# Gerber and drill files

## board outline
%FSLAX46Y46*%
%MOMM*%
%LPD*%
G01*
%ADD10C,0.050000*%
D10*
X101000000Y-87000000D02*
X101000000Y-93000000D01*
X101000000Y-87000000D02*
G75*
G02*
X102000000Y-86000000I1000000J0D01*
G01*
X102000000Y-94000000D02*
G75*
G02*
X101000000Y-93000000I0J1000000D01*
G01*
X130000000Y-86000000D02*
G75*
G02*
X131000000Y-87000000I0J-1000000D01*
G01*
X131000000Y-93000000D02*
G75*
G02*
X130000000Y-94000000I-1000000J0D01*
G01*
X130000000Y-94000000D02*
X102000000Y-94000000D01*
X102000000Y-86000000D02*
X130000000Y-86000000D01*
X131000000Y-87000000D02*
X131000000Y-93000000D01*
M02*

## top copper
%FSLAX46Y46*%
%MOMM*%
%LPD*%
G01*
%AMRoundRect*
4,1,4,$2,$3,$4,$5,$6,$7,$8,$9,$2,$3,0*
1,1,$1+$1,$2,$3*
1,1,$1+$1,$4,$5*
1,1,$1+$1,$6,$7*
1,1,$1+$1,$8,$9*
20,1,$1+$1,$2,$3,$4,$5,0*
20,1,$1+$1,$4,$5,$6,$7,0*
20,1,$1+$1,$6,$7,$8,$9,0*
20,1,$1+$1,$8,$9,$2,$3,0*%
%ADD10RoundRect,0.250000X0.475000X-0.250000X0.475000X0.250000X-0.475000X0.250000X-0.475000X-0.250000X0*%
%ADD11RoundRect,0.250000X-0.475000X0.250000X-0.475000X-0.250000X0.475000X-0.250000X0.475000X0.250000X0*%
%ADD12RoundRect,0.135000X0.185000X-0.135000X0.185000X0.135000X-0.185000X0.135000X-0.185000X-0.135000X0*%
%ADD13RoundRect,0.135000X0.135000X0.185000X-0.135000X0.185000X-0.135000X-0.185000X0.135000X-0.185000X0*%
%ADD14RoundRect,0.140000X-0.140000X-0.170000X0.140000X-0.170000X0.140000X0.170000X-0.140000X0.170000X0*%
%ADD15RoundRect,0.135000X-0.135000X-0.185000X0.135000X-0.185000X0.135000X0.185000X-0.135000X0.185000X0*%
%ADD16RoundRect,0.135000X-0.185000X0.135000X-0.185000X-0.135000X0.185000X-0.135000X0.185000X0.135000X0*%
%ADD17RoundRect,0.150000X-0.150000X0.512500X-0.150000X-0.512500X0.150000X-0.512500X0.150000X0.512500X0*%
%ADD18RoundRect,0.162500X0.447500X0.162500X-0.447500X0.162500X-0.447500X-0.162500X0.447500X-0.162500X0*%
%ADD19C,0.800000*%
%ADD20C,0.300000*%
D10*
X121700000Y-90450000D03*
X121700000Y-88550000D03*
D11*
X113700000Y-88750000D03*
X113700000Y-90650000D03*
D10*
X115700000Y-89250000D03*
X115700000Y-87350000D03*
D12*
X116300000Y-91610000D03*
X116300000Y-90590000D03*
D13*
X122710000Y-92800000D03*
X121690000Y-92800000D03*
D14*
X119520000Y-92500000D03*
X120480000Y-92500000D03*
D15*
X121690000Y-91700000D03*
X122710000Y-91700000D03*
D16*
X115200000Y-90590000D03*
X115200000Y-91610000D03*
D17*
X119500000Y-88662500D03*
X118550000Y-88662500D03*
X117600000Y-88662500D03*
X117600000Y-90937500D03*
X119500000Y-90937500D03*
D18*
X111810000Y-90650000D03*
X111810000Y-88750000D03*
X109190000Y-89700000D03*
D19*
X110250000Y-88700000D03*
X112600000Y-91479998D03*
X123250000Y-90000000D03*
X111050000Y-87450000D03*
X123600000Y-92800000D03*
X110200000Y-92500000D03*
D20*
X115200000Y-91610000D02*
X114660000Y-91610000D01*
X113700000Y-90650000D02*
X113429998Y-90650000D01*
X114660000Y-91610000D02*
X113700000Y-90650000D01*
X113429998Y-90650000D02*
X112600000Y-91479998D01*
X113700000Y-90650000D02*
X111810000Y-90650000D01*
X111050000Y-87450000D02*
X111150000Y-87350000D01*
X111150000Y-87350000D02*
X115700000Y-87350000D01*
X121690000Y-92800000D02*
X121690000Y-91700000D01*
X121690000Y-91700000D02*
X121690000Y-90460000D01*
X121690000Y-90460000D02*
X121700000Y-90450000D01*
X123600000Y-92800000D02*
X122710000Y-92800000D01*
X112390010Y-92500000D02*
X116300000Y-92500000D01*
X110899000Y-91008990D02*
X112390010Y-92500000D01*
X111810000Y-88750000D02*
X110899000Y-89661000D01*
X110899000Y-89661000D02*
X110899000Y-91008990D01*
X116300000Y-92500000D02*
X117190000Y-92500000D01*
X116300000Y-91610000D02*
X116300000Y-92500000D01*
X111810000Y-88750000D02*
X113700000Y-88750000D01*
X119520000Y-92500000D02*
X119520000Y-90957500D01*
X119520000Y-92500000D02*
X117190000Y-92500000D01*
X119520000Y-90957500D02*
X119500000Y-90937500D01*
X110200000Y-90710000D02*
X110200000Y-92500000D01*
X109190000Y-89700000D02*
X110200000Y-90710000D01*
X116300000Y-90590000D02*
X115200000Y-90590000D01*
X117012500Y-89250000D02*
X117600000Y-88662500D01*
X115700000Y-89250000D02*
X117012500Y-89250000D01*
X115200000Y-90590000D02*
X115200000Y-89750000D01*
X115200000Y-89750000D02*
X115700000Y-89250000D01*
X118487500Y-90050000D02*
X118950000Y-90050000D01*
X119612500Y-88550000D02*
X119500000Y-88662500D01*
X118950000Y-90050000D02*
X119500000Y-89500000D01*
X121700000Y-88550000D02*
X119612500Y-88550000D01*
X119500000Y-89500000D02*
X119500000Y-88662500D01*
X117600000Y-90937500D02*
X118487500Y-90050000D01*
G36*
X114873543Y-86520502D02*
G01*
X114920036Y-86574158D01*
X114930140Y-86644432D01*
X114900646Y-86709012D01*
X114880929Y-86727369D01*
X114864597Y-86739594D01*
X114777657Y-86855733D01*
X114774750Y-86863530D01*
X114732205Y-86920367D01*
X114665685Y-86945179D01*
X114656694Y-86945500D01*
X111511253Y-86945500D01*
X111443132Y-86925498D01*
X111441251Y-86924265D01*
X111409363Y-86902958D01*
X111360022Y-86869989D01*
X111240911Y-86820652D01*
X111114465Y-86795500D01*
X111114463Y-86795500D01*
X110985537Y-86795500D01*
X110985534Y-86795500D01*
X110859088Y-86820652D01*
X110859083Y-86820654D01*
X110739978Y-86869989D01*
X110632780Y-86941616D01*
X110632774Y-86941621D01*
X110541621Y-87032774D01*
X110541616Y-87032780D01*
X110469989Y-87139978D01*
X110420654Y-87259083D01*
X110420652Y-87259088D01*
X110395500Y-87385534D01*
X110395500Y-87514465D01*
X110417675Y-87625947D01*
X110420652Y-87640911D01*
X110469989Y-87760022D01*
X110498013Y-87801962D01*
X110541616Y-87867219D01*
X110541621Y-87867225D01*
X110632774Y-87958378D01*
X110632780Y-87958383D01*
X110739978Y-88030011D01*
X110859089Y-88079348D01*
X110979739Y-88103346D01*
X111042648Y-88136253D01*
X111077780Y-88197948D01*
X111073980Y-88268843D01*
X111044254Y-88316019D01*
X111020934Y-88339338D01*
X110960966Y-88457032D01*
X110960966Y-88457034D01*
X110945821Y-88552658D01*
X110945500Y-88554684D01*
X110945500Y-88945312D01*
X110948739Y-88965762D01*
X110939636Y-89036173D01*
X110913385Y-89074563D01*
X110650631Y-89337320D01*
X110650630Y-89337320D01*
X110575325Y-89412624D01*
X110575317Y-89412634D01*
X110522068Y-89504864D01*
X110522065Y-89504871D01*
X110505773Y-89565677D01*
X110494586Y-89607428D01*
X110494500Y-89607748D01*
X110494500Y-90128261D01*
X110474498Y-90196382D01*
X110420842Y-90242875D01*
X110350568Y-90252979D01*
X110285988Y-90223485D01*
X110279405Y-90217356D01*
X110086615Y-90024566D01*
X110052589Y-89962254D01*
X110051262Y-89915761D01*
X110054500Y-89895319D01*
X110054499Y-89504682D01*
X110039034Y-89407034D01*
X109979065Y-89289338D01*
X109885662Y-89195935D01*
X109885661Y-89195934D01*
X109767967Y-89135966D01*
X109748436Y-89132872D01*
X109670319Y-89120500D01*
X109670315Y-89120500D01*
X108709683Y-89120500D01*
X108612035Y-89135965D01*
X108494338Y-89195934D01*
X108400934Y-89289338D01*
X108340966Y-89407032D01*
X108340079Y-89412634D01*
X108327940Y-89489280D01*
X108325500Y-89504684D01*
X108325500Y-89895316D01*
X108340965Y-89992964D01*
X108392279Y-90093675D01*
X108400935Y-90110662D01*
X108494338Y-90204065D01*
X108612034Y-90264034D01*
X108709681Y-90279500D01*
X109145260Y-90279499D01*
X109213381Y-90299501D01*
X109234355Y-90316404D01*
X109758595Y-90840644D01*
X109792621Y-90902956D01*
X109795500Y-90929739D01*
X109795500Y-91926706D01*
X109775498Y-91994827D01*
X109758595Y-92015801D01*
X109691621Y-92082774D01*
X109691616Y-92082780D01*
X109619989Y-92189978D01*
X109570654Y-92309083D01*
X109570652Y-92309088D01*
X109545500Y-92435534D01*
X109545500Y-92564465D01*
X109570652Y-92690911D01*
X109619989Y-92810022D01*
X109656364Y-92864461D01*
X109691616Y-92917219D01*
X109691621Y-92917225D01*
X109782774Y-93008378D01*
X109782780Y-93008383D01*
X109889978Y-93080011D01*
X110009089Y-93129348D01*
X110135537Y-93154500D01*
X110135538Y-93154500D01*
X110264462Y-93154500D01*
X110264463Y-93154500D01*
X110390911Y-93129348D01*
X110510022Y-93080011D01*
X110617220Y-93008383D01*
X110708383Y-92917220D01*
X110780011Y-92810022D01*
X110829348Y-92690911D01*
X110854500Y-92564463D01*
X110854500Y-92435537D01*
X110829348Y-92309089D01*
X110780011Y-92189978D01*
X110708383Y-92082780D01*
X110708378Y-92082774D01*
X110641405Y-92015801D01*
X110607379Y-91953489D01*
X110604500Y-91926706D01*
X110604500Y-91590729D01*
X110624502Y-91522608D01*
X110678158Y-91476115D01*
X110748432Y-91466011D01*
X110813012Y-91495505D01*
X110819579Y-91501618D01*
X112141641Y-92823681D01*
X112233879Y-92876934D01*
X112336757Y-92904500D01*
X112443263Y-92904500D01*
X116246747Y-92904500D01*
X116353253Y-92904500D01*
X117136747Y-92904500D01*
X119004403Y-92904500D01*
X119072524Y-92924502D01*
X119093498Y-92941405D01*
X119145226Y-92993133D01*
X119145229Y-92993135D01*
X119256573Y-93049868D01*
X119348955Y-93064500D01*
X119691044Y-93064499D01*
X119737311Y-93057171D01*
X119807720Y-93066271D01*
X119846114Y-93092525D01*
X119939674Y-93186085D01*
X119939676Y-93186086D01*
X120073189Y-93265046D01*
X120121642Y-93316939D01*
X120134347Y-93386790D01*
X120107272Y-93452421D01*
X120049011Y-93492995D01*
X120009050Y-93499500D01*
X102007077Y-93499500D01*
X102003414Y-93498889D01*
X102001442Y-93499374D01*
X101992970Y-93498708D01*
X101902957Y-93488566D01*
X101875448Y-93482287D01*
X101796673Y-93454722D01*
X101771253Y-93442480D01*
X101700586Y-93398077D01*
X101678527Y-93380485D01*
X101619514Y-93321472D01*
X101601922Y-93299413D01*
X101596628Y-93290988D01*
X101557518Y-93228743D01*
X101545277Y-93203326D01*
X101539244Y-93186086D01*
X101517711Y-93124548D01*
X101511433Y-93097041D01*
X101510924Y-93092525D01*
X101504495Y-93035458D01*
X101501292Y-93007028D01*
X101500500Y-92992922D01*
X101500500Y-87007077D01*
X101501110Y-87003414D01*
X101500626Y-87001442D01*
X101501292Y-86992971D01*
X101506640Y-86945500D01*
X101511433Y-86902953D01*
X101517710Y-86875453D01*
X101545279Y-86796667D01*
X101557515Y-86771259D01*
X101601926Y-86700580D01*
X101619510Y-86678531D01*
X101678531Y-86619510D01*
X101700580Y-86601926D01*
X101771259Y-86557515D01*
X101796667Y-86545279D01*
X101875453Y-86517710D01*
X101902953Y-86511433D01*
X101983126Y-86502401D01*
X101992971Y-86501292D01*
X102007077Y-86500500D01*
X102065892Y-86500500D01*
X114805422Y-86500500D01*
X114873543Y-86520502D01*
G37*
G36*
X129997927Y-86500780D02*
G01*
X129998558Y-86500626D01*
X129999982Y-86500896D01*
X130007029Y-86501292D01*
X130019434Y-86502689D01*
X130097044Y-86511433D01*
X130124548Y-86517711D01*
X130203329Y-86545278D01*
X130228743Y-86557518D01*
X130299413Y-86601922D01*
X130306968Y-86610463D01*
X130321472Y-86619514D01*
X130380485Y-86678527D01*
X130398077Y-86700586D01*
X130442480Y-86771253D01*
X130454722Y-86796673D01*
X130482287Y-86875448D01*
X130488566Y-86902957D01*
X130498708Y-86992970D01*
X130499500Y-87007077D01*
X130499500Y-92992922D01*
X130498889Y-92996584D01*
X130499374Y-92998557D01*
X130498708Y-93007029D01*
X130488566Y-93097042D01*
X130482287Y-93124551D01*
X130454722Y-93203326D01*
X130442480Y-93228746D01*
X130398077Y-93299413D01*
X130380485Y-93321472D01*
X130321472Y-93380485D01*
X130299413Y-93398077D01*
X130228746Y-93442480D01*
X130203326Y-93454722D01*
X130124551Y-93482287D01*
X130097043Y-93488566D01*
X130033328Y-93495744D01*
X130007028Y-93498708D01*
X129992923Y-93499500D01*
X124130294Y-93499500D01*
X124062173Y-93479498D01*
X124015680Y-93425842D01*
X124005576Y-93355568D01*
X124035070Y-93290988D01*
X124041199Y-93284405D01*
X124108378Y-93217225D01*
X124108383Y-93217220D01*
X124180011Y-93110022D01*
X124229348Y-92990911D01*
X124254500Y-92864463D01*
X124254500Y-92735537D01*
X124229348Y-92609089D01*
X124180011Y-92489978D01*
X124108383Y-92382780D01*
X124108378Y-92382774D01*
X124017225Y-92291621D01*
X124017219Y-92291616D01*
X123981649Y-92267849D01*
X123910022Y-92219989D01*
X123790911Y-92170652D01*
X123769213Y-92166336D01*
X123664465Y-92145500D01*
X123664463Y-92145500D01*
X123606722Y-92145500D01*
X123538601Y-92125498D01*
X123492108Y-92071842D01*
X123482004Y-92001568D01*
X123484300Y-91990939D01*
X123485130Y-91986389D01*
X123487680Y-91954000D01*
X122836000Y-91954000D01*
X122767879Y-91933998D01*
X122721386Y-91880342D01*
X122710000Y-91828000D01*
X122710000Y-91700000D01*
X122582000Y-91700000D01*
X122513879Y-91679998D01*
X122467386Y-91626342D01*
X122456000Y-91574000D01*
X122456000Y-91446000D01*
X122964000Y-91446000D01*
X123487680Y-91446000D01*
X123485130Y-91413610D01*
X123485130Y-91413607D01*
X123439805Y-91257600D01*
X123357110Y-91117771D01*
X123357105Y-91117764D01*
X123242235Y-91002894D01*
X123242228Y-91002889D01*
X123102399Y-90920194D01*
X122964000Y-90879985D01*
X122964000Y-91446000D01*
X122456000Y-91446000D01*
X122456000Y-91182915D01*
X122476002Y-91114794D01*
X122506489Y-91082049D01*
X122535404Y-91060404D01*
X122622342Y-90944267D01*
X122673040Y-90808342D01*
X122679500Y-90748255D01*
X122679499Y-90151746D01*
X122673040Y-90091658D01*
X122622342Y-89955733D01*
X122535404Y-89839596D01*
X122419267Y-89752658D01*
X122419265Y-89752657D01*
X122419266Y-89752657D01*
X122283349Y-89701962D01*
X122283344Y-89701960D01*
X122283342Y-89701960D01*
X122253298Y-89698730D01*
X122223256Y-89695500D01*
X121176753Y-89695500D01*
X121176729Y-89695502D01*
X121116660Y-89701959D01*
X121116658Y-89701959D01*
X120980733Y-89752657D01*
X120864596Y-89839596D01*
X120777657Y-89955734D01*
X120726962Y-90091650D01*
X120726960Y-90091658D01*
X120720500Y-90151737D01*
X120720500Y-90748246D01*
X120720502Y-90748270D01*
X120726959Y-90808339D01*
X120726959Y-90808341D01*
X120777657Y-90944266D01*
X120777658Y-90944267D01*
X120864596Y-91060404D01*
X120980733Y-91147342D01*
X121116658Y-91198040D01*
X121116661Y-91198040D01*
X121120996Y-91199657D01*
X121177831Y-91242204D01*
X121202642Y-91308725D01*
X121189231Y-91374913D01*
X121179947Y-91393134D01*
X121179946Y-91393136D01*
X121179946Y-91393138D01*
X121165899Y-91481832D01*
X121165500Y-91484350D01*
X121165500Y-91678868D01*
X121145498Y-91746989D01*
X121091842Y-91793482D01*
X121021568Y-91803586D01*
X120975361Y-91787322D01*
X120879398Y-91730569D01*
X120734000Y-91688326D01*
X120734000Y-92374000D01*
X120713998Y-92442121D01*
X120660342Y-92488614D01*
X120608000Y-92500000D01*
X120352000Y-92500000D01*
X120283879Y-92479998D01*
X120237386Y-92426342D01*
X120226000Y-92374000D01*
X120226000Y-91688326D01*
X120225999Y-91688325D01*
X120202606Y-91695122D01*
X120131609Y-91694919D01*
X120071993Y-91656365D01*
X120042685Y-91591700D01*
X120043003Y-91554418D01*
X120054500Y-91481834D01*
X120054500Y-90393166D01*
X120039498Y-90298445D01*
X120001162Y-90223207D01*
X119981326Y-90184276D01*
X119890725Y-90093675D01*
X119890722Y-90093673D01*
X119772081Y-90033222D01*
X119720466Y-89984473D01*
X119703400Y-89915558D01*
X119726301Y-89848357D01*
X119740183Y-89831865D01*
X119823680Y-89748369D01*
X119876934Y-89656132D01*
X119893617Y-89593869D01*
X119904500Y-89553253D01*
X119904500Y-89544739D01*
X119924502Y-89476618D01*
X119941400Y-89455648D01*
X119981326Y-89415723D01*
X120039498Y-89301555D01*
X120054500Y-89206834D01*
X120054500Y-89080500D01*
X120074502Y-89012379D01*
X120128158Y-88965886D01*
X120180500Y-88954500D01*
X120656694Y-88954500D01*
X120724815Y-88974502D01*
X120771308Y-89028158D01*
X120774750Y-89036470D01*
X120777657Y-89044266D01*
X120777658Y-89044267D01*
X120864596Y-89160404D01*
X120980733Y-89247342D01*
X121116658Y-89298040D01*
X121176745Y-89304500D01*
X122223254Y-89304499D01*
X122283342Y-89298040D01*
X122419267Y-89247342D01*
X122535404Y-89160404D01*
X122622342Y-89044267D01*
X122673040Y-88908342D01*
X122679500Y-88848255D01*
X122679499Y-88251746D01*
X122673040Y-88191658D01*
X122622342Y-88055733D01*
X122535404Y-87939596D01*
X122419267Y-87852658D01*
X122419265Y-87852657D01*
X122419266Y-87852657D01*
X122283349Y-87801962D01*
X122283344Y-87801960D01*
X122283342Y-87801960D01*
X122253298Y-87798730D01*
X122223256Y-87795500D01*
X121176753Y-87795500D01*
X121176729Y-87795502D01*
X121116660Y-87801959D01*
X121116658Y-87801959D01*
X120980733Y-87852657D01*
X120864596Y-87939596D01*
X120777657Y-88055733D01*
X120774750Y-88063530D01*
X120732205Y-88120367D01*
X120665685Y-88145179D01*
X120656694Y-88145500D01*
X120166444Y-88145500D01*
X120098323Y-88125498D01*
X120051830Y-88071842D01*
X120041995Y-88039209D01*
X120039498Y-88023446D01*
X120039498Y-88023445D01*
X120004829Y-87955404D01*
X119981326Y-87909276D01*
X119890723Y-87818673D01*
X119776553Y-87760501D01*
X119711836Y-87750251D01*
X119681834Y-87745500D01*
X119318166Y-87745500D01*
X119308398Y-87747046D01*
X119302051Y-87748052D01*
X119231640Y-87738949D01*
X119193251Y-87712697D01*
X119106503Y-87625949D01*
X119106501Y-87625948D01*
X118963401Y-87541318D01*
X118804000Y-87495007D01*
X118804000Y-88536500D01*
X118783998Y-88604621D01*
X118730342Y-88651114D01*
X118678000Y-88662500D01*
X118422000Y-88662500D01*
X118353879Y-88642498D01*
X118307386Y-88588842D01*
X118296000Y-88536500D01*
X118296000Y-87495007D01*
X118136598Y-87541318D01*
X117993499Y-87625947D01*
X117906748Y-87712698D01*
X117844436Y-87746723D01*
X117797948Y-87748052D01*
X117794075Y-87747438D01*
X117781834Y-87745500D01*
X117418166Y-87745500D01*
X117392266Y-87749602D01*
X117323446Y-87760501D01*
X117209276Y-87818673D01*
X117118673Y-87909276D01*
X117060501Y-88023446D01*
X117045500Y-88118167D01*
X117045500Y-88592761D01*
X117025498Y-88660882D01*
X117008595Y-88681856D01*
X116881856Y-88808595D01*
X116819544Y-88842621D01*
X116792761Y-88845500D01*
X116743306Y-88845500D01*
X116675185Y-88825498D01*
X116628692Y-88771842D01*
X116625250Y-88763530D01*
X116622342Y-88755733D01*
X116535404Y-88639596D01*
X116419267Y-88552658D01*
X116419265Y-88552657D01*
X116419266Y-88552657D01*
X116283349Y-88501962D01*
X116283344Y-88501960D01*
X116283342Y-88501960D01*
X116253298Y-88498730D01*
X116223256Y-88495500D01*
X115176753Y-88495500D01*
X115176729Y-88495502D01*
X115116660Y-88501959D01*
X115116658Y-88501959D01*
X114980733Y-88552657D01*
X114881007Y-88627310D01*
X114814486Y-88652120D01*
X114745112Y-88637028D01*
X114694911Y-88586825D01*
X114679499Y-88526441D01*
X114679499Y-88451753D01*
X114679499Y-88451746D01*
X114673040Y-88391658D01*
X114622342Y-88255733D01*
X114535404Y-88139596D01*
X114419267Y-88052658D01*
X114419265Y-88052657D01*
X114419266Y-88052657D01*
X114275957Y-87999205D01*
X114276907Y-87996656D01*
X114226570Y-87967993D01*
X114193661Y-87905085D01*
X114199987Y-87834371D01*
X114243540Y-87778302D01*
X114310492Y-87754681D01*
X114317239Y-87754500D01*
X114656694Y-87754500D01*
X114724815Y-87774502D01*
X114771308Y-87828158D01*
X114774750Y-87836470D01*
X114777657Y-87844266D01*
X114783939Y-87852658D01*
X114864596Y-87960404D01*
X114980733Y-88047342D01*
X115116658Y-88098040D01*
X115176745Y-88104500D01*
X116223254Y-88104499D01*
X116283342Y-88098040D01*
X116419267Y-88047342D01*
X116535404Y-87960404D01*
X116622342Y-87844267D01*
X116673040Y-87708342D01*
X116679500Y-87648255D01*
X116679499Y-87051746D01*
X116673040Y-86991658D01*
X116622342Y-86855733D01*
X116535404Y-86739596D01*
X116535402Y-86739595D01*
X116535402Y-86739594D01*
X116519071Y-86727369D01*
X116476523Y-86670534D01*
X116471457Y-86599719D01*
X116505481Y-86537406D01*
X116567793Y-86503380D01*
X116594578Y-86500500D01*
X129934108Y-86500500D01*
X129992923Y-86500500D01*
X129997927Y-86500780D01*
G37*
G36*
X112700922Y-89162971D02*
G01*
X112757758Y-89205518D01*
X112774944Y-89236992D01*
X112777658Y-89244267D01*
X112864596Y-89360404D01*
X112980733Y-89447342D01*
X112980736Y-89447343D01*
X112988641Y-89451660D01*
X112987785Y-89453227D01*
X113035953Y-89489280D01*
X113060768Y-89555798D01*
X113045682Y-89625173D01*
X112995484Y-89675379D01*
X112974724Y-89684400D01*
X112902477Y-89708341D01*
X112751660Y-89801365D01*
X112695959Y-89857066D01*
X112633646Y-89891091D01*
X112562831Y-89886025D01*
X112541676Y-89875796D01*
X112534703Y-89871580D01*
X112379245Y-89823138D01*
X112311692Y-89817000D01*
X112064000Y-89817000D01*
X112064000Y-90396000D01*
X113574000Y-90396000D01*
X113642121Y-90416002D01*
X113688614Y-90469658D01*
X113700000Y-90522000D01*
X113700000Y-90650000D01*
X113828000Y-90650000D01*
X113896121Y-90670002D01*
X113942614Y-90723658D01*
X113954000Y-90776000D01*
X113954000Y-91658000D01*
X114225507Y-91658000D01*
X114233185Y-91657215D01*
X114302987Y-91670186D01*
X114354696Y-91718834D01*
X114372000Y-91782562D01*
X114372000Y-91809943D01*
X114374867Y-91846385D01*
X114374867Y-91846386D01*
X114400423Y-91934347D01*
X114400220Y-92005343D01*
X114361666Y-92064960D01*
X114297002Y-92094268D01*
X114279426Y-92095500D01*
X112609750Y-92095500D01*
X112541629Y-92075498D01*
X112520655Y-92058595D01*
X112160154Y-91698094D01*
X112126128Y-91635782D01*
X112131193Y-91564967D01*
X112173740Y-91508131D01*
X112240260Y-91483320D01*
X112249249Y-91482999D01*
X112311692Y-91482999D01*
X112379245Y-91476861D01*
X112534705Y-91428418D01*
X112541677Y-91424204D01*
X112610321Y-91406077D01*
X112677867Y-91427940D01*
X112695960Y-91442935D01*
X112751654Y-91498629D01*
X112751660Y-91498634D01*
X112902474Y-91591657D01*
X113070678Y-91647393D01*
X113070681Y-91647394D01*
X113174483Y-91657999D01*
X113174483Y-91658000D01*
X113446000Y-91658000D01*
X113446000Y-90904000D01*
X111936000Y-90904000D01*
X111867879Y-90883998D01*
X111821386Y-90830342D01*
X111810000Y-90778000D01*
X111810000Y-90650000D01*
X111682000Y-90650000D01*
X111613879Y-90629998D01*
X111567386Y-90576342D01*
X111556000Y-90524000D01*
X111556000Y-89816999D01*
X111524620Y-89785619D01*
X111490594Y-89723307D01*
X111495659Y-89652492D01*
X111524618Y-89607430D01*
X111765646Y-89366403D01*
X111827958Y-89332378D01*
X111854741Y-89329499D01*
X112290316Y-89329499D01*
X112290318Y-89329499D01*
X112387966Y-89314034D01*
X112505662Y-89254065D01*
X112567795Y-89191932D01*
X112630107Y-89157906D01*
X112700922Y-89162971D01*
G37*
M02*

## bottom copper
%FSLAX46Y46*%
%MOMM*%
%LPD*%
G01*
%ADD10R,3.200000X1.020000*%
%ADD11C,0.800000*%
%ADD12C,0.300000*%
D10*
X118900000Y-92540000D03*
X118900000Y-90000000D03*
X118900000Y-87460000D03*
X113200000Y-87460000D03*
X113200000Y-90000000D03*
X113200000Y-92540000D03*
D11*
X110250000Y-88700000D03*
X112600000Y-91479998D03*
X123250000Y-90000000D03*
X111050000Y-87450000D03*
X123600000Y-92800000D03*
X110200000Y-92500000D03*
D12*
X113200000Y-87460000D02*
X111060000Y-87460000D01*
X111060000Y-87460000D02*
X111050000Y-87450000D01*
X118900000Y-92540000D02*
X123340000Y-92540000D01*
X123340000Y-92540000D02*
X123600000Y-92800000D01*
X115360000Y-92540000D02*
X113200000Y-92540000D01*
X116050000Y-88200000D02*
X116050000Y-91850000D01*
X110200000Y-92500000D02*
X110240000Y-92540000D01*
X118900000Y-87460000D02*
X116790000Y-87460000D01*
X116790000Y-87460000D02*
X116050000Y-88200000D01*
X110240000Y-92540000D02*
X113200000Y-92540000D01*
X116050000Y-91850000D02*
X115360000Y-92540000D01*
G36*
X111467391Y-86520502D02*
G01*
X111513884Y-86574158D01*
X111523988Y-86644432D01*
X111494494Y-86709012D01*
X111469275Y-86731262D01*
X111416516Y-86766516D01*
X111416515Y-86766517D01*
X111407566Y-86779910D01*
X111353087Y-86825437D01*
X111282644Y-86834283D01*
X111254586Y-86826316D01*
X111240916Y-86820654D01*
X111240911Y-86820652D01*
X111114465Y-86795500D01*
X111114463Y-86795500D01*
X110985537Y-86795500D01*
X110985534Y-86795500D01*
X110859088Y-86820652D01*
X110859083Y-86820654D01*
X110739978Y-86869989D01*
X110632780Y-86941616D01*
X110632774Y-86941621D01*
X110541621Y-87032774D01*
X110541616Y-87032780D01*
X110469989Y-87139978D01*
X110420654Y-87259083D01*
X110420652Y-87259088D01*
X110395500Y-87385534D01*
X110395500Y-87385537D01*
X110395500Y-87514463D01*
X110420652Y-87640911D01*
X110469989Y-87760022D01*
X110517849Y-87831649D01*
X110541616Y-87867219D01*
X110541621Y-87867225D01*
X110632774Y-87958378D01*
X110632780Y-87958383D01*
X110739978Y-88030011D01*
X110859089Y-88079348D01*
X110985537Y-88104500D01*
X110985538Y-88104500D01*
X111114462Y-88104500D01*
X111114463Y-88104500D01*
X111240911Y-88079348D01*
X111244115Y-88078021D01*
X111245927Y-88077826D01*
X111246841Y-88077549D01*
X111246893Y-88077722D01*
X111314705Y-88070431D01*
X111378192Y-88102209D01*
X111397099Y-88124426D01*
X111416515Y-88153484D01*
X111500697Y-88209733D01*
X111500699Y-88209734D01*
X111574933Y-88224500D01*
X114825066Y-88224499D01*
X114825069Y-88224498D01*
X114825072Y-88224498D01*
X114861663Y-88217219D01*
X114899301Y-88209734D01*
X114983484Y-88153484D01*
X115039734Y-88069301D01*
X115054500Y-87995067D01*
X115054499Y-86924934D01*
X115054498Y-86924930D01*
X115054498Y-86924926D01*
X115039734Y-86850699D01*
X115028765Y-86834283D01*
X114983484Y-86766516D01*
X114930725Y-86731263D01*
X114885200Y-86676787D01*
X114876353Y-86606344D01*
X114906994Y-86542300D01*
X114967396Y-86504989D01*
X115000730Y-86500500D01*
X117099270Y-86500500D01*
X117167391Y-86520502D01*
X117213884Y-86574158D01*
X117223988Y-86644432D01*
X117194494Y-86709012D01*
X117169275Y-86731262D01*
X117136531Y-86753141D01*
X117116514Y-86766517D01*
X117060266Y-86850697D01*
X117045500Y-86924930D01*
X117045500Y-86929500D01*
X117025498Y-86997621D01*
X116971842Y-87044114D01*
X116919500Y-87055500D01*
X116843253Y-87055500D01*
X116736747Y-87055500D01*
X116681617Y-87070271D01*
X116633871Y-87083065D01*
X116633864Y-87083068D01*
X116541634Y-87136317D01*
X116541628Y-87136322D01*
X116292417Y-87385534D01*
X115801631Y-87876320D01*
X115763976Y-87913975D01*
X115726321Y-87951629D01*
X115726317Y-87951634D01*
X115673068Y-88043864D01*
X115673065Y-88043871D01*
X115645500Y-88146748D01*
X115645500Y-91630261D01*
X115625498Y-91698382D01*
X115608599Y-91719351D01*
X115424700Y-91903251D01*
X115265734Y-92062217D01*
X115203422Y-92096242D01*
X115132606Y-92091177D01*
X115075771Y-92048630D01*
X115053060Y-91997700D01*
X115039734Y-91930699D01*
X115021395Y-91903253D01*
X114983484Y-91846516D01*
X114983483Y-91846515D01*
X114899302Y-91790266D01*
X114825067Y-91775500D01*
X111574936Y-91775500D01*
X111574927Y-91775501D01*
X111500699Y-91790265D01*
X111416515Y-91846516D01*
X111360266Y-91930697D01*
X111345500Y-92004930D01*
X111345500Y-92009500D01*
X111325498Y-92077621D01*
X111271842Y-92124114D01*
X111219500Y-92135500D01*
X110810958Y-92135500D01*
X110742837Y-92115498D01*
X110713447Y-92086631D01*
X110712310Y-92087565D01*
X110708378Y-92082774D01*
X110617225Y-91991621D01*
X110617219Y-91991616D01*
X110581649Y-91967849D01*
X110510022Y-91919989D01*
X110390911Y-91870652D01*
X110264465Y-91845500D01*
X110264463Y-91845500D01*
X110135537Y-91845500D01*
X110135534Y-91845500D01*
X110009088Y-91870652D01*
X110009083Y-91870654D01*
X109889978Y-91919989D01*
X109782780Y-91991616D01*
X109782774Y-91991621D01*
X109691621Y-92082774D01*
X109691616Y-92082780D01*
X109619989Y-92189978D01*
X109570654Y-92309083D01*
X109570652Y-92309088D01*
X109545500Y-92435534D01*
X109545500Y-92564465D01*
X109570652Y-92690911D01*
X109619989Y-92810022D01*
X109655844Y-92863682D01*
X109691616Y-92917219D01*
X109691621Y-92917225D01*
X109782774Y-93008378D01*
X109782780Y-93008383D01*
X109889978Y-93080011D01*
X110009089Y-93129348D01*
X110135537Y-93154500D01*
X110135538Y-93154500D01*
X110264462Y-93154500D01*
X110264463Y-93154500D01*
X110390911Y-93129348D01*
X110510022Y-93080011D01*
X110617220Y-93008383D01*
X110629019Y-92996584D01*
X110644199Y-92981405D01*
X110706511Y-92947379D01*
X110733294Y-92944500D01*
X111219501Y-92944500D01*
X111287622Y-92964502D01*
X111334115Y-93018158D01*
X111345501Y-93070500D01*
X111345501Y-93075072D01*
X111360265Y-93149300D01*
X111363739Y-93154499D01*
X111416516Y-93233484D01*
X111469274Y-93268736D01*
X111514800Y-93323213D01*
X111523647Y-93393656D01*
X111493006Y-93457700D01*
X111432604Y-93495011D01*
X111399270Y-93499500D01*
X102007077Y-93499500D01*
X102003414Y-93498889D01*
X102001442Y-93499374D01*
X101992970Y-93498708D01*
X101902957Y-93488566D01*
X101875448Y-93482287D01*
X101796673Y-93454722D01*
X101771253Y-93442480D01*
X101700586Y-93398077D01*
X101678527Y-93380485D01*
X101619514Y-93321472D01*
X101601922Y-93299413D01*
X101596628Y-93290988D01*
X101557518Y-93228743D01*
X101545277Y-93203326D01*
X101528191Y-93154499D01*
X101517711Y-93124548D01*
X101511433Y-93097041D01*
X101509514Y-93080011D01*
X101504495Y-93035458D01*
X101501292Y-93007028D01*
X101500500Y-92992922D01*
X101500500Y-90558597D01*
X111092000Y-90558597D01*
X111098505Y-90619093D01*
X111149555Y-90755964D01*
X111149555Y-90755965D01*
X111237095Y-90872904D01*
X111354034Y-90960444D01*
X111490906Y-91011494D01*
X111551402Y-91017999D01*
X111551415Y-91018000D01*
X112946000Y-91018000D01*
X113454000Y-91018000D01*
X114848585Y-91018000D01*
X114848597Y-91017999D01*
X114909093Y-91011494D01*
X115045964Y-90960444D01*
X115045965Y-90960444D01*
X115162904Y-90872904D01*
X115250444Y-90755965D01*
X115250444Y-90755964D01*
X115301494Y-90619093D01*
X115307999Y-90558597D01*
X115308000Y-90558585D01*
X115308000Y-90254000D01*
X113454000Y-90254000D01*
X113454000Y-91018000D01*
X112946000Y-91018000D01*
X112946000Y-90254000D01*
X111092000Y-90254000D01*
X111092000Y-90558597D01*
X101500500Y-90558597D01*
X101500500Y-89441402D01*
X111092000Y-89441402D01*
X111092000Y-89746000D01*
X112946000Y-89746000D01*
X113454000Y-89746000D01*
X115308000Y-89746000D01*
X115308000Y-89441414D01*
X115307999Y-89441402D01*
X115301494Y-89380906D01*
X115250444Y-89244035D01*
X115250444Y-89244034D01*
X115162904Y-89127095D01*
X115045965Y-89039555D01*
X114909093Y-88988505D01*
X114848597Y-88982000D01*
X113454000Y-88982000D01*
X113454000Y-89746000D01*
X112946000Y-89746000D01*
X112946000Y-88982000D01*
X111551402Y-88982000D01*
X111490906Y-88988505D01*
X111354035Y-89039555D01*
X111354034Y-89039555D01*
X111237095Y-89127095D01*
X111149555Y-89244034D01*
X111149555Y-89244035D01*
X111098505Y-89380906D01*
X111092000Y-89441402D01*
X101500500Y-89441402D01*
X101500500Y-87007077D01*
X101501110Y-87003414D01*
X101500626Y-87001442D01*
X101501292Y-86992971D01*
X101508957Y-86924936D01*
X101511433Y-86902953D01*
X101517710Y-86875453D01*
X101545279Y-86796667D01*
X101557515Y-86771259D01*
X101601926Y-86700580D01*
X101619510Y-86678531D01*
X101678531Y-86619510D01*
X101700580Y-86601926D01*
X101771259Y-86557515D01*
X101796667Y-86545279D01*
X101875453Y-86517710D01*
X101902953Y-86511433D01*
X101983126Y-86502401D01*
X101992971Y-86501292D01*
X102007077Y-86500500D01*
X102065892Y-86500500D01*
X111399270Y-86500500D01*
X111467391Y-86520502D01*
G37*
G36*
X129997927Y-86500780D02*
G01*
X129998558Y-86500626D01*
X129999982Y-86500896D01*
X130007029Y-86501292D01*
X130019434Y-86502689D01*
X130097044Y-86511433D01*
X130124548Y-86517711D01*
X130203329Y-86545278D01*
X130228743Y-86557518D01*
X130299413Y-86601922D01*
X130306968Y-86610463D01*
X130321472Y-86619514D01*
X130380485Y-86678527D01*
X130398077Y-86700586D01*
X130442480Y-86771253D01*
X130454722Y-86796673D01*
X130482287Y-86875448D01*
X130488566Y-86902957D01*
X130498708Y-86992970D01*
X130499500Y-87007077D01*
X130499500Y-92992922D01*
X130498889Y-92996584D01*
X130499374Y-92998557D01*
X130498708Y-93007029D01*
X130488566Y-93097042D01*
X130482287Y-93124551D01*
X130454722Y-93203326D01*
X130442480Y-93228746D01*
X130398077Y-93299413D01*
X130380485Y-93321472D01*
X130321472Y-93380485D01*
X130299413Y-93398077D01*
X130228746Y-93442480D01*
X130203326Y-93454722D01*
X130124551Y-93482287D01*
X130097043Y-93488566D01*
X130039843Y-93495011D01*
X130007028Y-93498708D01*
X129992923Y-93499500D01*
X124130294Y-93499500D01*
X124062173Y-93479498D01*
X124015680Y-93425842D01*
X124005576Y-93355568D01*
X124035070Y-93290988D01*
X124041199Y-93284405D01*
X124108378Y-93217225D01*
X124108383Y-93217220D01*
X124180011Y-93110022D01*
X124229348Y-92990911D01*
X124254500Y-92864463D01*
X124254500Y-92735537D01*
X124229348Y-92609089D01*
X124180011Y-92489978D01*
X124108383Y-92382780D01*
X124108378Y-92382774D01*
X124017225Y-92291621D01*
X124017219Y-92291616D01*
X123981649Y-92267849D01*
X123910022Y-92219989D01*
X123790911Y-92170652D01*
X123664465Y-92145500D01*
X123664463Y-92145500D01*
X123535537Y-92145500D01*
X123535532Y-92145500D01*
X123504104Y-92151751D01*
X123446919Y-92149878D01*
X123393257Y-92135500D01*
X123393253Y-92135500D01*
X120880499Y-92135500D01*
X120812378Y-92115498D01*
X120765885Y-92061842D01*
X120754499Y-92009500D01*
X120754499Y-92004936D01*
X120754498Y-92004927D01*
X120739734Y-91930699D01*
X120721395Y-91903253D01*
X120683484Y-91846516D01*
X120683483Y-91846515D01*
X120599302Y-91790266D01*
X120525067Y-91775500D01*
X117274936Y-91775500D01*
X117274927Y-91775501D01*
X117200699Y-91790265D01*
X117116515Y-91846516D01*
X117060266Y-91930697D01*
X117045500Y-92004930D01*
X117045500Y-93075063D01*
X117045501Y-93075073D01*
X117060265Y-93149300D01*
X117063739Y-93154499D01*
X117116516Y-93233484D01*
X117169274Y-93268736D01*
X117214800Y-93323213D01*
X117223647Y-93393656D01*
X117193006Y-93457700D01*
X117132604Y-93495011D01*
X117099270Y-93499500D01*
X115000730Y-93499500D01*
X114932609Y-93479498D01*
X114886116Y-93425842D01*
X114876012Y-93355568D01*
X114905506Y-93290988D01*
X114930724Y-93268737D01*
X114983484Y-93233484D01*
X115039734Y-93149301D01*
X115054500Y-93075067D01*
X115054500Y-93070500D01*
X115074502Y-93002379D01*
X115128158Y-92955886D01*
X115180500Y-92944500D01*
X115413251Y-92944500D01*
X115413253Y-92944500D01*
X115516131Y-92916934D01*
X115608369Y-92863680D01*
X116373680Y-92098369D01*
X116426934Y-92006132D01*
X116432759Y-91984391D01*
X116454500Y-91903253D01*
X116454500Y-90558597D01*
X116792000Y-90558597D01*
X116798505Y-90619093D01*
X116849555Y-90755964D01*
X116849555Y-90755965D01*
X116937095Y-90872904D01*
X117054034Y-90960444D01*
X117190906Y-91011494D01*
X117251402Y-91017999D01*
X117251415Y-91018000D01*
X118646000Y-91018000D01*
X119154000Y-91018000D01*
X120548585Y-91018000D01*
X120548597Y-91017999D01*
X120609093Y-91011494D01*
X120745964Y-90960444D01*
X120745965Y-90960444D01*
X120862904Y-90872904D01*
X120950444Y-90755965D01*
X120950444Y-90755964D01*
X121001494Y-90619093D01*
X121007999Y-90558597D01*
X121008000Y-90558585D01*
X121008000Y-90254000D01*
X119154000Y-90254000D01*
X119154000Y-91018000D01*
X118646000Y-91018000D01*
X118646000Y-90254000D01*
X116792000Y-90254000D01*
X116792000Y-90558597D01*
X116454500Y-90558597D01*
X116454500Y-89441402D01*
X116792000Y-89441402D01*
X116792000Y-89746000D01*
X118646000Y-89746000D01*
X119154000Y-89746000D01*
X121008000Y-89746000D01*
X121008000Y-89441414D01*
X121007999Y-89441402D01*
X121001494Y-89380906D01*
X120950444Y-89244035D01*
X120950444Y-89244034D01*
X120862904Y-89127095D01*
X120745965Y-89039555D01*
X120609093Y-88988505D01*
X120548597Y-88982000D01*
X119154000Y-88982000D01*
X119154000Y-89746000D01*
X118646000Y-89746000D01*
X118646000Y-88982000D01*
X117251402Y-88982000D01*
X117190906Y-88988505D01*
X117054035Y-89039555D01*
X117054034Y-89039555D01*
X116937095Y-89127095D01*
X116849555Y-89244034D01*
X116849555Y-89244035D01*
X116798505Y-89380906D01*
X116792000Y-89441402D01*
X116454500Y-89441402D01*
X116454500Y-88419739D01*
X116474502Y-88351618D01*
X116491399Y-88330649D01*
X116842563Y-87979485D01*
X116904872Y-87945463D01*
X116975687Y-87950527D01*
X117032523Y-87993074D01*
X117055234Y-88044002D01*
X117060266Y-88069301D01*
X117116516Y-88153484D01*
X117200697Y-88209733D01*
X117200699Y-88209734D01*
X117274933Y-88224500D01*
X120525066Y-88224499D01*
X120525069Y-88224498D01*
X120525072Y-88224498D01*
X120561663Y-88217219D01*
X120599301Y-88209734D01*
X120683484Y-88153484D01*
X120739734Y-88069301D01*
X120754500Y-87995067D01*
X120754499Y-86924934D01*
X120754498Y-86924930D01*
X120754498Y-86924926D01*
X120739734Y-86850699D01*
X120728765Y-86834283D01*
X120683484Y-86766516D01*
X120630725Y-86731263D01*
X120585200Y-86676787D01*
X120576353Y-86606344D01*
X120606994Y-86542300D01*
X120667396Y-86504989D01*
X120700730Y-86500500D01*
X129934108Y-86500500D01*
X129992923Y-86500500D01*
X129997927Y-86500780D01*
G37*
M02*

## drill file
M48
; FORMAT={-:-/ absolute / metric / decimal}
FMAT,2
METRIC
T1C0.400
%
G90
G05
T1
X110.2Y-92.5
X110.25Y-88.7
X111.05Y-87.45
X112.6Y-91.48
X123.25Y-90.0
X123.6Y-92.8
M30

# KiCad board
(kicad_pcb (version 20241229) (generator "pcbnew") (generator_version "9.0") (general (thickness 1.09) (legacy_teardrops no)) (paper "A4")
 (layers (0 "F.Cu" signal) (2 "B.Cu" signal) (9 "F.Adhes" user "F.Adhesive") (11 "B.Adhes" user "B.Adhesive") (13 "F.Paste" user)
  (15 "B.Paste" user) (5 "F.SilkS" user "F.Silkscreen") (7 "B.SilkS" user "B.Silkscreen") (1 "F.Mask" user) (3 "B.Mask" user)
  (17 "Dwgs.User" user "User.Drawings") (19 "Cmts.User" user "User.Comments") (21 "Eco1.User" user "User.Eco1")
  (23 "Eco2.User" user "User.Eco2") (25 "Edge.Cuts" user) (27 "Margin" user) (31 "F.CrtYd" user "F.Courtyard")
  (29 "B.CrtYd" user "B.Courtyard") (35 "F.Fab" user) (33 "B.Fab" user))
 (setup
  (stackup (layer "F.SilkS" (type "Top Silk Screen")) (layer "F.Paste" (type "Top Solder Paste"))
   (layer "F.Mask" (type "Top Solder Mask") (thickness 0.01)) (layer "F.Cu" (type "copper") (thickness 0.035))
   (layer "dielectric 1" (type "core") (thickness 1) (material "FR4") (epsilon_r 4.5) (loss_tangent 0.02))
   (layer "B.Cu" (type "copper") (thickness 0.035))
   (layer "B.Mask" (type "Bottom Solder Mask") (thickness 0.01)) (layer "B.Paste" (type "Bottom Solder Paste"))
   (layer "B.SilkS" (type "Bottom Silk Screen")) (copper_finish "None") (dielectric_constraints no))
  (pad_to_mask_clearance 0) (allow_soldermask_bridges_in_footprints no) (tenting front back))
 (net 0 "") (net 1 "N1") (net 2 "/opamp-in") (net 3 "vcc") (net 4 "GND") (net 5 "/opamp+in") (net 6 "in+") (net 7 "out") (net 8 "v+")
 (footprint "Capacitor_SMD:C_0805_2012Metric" (layer "F.Cu") (at 121.7 89.5 90)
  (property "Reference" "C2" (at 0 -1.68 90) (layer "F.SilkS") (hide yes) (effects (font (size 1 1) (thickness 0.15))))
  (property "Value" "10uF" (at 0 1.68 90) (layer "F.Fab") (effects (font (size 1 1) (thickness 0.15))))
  (pad "1" smd roundrect (at -0.95 0 90) (size 1 1.45) (layers "F.Cu" "F.Mask" "F.Paste") (roundrect_rratio 0.25) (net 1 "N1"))
  (pad "2" smd roundrect (at 0.95 0 90) (size 1 1.45) (layers "F.Cu" "F.Mask" "F.Paste") (roundrect_rratio 0.25) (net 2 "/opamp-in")))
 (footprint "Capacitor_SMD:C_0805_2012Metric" (layer "F.Cu") (at 113.7 89.7 -90)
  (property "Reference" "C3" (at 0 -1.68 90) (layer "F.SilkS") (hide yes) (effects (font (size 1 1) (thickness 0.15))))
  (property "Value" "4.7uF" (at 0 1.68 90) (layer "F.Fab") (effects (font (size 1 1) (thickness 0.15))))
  (pad "1" smd roundrect (at -0.95 0 270) (size 1 1.45) (layers "F.Cu" "F.Mask" "F.Paste") (roundrect_rratio 0.25) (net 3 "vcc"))
  (pad "2" smd roundrect (at 0.95 0 270) (size 1 1.45) (layers "F.Cu" "F.Mask" "F.Paste") (roundrect_rratio 0.25) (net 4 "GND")))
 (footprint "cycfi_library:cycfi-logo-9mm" (layer "F.Cu") (at 125.9 86.9)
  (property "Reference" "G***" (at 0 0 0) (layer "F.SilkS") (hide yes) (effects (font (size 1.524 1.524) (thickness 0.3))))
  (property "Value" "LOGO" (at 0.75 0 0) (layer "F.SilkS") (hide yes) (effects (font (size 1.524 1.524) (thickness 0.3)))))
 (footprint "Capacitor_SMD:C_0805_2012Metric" (layer "F.Cu") (at 115.7 88.3 90)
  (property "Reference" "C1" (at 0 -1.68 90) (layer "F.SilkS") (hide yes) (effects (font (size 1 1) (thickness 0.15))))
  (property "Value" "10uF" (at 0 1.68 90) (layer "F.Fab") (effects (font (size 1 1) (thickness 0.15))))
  (pad "1" smd roundrect (at -0.95 0 90) (size 1 1.45) (layers "F.Cu" "F.Mask" "F.Paste") (roundrect_rratio 0.25) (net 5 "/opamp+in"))
  (pad "2" smd roundrect (at 0.95 0 90) (size 1 1.45) (layers "F.Cu" "F.Mask" "F.Paste") (roundrect_rratio 0.25) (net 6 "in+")))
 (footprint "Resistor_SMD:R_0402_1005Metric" (layer "F.Cu") (at 116.3 91.1 90)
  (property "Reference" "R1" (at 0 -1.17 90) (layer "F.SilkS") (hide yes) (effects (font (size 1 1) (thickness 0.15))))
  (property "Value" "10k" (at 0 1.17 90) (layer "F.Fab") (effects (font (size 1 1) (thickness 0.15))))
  (pad "1" smd roundrect (at -0.51 0 90) (size 0.54 0.64) (layers "F.Cu" "F.Mask" "F.Paste") (roundrect_rratio 0.25) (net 3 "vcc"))
  (pad "2" smd roundrect (at 0.51 0 90) (size 0.54 0.64) (layers "F.Cu" "F.Mask" "F.Paste") (roundrect_rratio 0.25) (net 5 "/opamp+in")))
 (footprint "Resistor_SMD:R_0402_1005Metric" (layer "F.Cu") (at 122.2 92.8 180)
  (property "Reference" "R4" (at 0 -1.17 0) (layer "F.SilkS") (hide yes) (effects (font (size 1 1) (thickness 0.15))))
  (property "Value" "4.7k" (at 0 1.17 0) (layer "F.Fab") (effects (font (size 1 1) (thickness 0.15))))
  (pad "1" smd roundrect (at -0.51 0 180) (size 0.54 0.64) (layers "F.Cu" "F.Mask" "F.Paste") (roundrect_rratio 0.25) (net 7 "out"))
  (pad "2" smd roundrect (at 0.51 0 180) (size 0.54 0.64) (layers "F.Cu" "F.Mask" "F.Paste") (roundrect_rratio 0.25) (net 1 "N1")))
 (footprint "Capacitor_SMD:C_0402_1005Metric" (layer "F.Cu") (at 120 92.5)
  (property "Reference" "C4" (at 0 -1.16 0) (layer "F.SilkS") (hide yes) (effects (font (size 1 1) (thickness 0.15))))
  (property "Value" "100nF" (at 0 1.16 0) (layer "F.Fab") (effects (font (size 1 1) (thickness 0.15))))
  (pad "1" smd roundrect (at -0.48 0) (size 0.56 0.62) (layers "F.Cu" "F.Mask" "F.Paste") (roundrect_rratio 0.25) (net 3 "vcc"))
  (pad "2" smd roundrect (at 0.48 0) (size 0.56 0.62) (layers "F.Cu" "F.Mask" "F.Paste") (roundrect_rratio 0.25) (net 4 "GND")))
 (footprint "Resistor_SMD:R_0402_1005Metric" (layer "F.Cu") (at 122.2 91.7)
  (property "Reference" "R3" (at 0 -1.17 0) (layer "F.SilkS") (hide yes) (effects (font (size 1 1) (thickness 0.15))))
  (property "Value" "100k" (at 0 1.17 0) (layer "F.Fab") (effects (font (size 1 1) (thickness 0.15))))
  (pad "1" smd roundrect (at -0.51 0) (size 0.54 0.64) (layers "F.Cu" "F.Mask" "F.Paste") (roundrect_rratio 0.25) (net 1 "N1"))
  (pad "2" smd roundrect (at 0.51 0) (size 0.54 0.64) (layers "F.Cu" "F.Mask" "F.Paste") (roundrect_rratio 0.25) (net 4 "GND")))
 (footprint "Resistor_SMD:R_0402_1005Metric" (layer "F.Cu") (at 115.2 91.1 -90)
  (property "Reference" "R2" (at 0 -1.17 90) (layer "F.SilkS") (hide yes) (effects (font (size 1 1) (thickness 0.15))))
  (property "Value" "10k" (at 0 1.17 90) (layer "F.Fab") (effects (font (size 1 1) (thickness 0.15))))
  (pad "1" smd roundrect (at -0.51 0 270) (size 0.54 0.64) (layers "F.Cu" "F.Mask" "F.Paste") (roundrect_rratio 0.25) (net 5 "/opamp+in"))
  (pad "2" smd roundrect (at 0.51 0 270) (size 0.54 0.64) (layers "F.Cu" "F.Mask" "F.Paste") (roundrect_rratio 0.25) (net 4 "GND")))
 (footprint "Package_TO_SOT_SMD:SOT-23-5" (layer "F.Cu") (at 118.55 89.8 -90)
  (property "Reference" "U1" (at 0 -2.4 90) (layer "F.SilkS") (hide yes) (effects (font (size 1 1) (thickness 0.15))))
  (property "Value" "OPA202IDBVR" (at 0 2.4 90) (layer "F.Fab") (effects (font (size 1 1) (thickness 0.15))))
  (pad "1" smd roundrect (at -1.1375 -0.95 270) (size 1.325 0.6) (layers "F.Cu" "F.Mask" "F.Paste") (roundrect_rratio 0.25)
   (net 2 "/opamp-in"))
  (pad "2" smd roundrect (at -1.1375 0 270) (size 1.325 0.6) (layers "F.Cu" "F.Mask" "F.Paste") (roundrect_rratio 0.25) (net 4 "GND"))
  (pad "3" smd roundrect (at -1.1375 0.95 270) (size 1.325 0.6) (layers "F.Cu" "F.Mask" "F.Paste") (roundrect_rratio 0.25)
   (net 5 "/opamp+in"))
  (pad "4" smd roundrect (at 1.1375 0.95 270) (size 1.325 0.6) (layers "F.Cu" "F.Mask" "F.Paste") (roundrect_rratio 0.25)
   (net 2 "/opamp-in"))
  (pad "5" smd roundrect (at 1.1375 -0.95 270) (size 1.325 0.6) (layers "F.Cu" "F.Mask" "F.Paste") (roundrect_rratio 0.25) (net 3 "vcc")))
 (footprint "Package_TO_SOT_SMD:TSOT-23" (layer "F.Cu") (at 110.5 89.7 180)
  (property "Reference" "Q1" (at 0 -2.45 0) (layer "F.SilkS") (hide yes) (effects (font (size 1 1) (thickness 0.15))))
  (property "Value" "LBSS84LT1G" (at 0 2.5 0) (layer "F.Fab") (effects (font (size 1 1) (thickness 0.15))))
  (pad "1" smd roundrect (at -1.31 -0.95 180) (size 1.22 0.65) (layers "F.Cu" "F.Mask" "F.Paste") (roundrect_rratio 0.25) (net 4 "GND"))
  (pad "2" smd roundrect (at -1.31 0.95 180) (size 1.22 0.65) (layers "F.Cu" "F.Mask" "F.Paste") (roundrect_rratio 0.25) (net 3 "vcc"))
  (pad "3" smd roundrect (at 1.31 0 180) (size 1.22 0.65) (layers "F.Cu" "F.Mask" "F.Paste") (roundrect_rratio 0.25) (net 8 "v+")))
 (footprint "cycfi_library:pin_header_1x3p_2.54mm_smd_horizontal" (layer "B.Cu") (at 118.9 92.54)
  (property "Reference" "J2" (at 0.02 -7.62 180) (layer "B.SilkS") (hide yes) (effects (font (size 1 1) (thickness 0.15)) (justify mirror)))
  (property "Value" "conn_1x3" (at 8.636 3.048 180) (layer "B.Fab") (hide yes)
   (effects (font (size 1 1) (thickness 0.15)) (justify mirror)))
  (pad "1" smd rect (at 0 0) (size 3.2 1.02) (layers "B.Cu" "B.Mask" "B.Paste") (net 7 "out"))
  (pad "2" smd rect (at 0 -2.54) (size 3.2 1.02) (layers "B.Cu" "B.Mask" "B.Paste") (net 4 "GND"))
  (pad "3" smd rect (at 0 -5.08) (size 3.2 1.02) (layers "B.Cu" "B.Mask" "B.Paste") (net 8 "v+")))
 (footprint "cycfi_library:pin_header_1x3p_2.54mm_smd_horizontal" (layer "B.Cu") (at 113.2 87.46 180)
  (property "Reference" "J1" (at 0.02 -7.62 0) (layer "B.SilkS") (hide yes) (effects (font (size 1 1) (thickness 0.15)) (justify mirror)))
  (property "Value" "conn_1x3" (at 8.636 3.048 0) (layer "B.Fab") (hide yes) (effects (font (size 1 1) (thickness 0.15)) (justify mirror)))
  (pad "1" smd rect (at 0 0 180) (size 3.2 1.02) (layers "B.Cu" "B.Mask" "B.Paste") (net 6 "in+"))
  (pad "2" smd rect (at 0 -2.54 180) (size 3.2 1.02) (layers "B.Cu" "B.Mask" "B.Paste") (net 4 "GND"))
  (pad "3" smd rect (at 0 -5.08 180) (size 3.2 1.02) (layers "B.Cu" "B.Mask" "B.Paste") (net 8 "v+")))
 (gr_line (start 101 87) (end 101 93) (stroke (width 0.05) (type solid)) (layer "Edge.Cuts"))
 (gr_arc (start 101 87) (mid 101.292893 86.292893) (end 102 86) (stroke (width 0.05) (type solid)) (layer "Edge.Cuts"))
 (gr_arc (start 102 94) (mid 101.292893 93.707107) (end 101 93) (stroke (width 0.05) (type solid)) (layer "Edge.Cuts"))
 (gr_arc (start 130 86) (mid 130.707107 86.292893) (end 131 87) (stroke (width 0.05) (type solid)) (layer "Edge.Cuts"))
 (gr_arc (start 131 93) (mid 130.707107 93.707107) (end 130 94) (stroke (width 0.05) (type solid)) (layer "Edge.Cuts"))
 (gr_line (start 130 94) (end 102 94) (stroke (width 0.05) (type solid)) (layer "Edge.Cuts"))
 (gr_line (start 102 86) (end 130 86) (stroke (width 0.05) (type solid)) (layer "Edge.Cuts"))
 (gr_line (start 131 87) (end 131 93) (stroke (width 0.05) (type solid)) (layer "Edge.Cuts"))
 (segment (start 115.2 91.61) (end 114.66 91.61) (width 0.3) (layer "F.Cu") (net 4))
 (segment (start 113.7 90.65) (end 113.429998 90.65) (width 0.3) (layer "F.Cu") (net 4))
 (segment (start 114.66 91.61) (end 113.7 90.65) (width 0.3) (layer "F.Cu") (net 4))
 (segment (start 113.429998 90.65) (end 112.6 91.479998) (width 0.3) (layer "F.Cu") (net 4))
 (segment (start 113.7 90.65) (end 111.81 90.65) (width 0.3) (layer "F.Cu") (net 4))
 (via (at 110.25 88.7) (size 0.8) (drill 0.4) (layers "F.Cu" "B.Cu") (free yes) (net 4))
 (via (at 112.6 91.479998) (size 0.8) (drill 0.4) (layers "F.Cu" "B.Cu") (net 4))
 (via (at 123.25 90) (size 0.8) (drill 0.4) (layers "F.Cu" "B.Cu") (free yes) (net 4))
 (segment (start 111.05 87.45) (end 111.15 87.35) (width 0.3) (layer "F.Cu") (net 6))
 (segment (start 111.15 87.35) (end 115.7 87.35) (width 0.3) (layer "F.Cu") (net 6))
 (via (at 111.05 87.45) (size 0.8) (drill 0.4) (layers "F.Cu" "B.Cu") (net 6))
 (segment (start 113.2 87.46) (end 111.06 87.46) (width 0.3) (layer "B.Cu") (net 6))
 (segment (start 111.06 87.46) (end 111.05 87.45) (width 0.3) (layer "B.Cu") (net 6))
 (segment (start 121.69 92.8) (end 121.69 91.7) (width 0.3) (layer "F.Cu") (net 1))
 (segment (start 121.69 91.7) (end 121.69 90.46) (width 0.3) (layer "F.Cu") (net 1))
 (segment (start 121.69 90.46) (end 121.7 90.45) (width 0.3) (layer "F.Cu") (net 1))
 (segment (start 123.6 92.8) (end 122.71 92.8) (width 0.3) (layer "F.Cu") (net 7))
 (via (at 123.6 92.8) (size 0.8) (drill 0.4) (layers "F.Cu" "B.Cu") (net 7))
 (segment (start 118.9 92.54) (end 123.34 92.54) (width 0.3) (layer "B.Cu") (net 7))
 (segment (start 123.34 92.54) (end 123.6 92.8) (width 0.3) (layer "B.Cu") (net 7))
 (segment (start 112.39001 92.5) (end 116.3 92.5) (width 0.3) (layer "F.Cu") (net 3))
 (segment (start 110.899 91.00899) (end 112.39001 92.5) (width 0.3) (layer "F.Cu") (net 3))
 (segment (start 111.81 88.75) (end 110.899 89.661) (width 0.3) (layer "F.Cu") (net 3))
 (segment (start 110.899 89.661) (end 110.899 91.00899) (width 0.3) (layer "F.Cu") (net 3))
 (segment (start 116.3 92.5) (end 117.19 92.5) (width 0.3) (layer "F.Cu") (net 3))
 (segment (start 116.3 91.61) (end 116.3 92.5) (width 0.3) (layer "F.Cu") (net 3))
 (segment (start 111.81 88.75) (end 113.7 88.75) (width 0.3) (layer "F.Cu") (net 3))
 (segment (start 119.52 92.5) (end 119.52 90.9575) (width 0.3) (layer "F.Cu") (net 3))
 (segment (start 119.52 92.5) (end 117.19 92.5) (width 0.3) (layer "F.Cu") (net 3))
 (segment (start 119.52 90.9575) (end 119.5 90.9375) (width 0.3) (layer "F.Cu") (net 3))
 (segment (start 110.2 90.71) (end 110.2 92.5) (width 0.3) (layer "F.Cu") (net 8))
 (segment (start 109.19 89.7) (end 110.2 90.71) (width 0.3) (layer "F.Cu") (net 8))
 (via (at 110.2 92.5) (size 0.8) (drill 0.4) (layers "F.Cu" "B.Cu") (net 8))
 (segment (start 115.36 92.54) (end 113.2 92.54) (width 0.3) (layer "B.Cu") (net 8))
 (segment (start 116.05 88.2) (end 116.05 91.85) (width 0.3) (layer "B.Cu") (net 8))
 (segment (start 110.2 92.5) (end 110.24 92.54) (width 0.3) (layer "B.Cu") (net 8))
 (segment (start 118.9 87.46) (end 116.79 87.46) (width 0.3) (layer "B.Cu") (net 8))
 (segment (start 116.79 87.46) (end 116.05 88.2) (width 0.3) (layer "B.Cu") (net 8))
 (segment (start 110.24 92.54) (end 113.2 92.54) (width 0.3) (layer "B.Cu") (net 8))
 (segment (start 116.05 91.85) (end 115.36 92.54) (width 0.3) (layer "B.Cu") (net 8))
 (segment (start 116.3 90.59) (end 115.2 90.59) (width 0.3) (layer "F.Cu") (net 5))
 (segment (start 117.0125 89.25) (end 117.6 88.6625) (width 0.3) (layer "F.Cu") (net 5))
 (segment (start 115.7 89.25) (end 117.0125 89.25) (width 0.3) (layer "F.Cu") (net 5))
 (segment (start 115.2 90.59) (end 115.2 89.75) (width 0.3) (layer "F.Cu") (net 5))
 (segment (start 115.2 89.75) (end 115.7 89.25) (width 0.3) (layer "F.Cu") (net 5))
 (segment (start 118.4875 90.05) (end 118.95 90.05) (width 0.3) (layer "F.Cu") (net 2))
 (segment (start 119.6125 88.55) (end 119.5 88.6625) (width 0.3) (layer "F.Cu") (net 2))
 (segment (start 118.95 90.05) (end 119.5 89.5) (width 0.3) (layer "F.Cu") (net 2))
 (segment (start 121.7 88.55) (end 119.6125 88.55) (width 0.3) (layer "F.Cu") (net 2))
 (segment (start 119.5 89.5) (end 119.5 88.6625) (width 0.3) (layer "F.Cu") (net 2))
 (segment (start 117.6 90.9375) (end 118.4875 90.05) (width 0.3) (layer "F.Cu") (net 2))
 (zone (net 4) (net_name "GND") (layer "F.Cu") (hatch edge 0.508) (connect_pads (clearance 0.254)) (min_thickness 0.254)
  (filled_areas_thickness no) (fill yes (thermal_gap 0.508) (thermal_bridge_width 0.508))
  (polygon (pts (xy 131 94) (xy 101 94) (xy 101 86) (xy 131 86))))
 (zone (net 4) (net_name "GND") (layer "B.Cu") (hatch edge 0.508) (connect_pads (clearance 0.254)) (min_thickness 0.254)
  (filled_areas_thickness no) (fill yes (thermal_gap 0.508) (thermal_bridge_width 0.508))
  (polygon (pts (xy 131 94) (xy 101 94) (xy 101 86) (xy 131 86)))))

